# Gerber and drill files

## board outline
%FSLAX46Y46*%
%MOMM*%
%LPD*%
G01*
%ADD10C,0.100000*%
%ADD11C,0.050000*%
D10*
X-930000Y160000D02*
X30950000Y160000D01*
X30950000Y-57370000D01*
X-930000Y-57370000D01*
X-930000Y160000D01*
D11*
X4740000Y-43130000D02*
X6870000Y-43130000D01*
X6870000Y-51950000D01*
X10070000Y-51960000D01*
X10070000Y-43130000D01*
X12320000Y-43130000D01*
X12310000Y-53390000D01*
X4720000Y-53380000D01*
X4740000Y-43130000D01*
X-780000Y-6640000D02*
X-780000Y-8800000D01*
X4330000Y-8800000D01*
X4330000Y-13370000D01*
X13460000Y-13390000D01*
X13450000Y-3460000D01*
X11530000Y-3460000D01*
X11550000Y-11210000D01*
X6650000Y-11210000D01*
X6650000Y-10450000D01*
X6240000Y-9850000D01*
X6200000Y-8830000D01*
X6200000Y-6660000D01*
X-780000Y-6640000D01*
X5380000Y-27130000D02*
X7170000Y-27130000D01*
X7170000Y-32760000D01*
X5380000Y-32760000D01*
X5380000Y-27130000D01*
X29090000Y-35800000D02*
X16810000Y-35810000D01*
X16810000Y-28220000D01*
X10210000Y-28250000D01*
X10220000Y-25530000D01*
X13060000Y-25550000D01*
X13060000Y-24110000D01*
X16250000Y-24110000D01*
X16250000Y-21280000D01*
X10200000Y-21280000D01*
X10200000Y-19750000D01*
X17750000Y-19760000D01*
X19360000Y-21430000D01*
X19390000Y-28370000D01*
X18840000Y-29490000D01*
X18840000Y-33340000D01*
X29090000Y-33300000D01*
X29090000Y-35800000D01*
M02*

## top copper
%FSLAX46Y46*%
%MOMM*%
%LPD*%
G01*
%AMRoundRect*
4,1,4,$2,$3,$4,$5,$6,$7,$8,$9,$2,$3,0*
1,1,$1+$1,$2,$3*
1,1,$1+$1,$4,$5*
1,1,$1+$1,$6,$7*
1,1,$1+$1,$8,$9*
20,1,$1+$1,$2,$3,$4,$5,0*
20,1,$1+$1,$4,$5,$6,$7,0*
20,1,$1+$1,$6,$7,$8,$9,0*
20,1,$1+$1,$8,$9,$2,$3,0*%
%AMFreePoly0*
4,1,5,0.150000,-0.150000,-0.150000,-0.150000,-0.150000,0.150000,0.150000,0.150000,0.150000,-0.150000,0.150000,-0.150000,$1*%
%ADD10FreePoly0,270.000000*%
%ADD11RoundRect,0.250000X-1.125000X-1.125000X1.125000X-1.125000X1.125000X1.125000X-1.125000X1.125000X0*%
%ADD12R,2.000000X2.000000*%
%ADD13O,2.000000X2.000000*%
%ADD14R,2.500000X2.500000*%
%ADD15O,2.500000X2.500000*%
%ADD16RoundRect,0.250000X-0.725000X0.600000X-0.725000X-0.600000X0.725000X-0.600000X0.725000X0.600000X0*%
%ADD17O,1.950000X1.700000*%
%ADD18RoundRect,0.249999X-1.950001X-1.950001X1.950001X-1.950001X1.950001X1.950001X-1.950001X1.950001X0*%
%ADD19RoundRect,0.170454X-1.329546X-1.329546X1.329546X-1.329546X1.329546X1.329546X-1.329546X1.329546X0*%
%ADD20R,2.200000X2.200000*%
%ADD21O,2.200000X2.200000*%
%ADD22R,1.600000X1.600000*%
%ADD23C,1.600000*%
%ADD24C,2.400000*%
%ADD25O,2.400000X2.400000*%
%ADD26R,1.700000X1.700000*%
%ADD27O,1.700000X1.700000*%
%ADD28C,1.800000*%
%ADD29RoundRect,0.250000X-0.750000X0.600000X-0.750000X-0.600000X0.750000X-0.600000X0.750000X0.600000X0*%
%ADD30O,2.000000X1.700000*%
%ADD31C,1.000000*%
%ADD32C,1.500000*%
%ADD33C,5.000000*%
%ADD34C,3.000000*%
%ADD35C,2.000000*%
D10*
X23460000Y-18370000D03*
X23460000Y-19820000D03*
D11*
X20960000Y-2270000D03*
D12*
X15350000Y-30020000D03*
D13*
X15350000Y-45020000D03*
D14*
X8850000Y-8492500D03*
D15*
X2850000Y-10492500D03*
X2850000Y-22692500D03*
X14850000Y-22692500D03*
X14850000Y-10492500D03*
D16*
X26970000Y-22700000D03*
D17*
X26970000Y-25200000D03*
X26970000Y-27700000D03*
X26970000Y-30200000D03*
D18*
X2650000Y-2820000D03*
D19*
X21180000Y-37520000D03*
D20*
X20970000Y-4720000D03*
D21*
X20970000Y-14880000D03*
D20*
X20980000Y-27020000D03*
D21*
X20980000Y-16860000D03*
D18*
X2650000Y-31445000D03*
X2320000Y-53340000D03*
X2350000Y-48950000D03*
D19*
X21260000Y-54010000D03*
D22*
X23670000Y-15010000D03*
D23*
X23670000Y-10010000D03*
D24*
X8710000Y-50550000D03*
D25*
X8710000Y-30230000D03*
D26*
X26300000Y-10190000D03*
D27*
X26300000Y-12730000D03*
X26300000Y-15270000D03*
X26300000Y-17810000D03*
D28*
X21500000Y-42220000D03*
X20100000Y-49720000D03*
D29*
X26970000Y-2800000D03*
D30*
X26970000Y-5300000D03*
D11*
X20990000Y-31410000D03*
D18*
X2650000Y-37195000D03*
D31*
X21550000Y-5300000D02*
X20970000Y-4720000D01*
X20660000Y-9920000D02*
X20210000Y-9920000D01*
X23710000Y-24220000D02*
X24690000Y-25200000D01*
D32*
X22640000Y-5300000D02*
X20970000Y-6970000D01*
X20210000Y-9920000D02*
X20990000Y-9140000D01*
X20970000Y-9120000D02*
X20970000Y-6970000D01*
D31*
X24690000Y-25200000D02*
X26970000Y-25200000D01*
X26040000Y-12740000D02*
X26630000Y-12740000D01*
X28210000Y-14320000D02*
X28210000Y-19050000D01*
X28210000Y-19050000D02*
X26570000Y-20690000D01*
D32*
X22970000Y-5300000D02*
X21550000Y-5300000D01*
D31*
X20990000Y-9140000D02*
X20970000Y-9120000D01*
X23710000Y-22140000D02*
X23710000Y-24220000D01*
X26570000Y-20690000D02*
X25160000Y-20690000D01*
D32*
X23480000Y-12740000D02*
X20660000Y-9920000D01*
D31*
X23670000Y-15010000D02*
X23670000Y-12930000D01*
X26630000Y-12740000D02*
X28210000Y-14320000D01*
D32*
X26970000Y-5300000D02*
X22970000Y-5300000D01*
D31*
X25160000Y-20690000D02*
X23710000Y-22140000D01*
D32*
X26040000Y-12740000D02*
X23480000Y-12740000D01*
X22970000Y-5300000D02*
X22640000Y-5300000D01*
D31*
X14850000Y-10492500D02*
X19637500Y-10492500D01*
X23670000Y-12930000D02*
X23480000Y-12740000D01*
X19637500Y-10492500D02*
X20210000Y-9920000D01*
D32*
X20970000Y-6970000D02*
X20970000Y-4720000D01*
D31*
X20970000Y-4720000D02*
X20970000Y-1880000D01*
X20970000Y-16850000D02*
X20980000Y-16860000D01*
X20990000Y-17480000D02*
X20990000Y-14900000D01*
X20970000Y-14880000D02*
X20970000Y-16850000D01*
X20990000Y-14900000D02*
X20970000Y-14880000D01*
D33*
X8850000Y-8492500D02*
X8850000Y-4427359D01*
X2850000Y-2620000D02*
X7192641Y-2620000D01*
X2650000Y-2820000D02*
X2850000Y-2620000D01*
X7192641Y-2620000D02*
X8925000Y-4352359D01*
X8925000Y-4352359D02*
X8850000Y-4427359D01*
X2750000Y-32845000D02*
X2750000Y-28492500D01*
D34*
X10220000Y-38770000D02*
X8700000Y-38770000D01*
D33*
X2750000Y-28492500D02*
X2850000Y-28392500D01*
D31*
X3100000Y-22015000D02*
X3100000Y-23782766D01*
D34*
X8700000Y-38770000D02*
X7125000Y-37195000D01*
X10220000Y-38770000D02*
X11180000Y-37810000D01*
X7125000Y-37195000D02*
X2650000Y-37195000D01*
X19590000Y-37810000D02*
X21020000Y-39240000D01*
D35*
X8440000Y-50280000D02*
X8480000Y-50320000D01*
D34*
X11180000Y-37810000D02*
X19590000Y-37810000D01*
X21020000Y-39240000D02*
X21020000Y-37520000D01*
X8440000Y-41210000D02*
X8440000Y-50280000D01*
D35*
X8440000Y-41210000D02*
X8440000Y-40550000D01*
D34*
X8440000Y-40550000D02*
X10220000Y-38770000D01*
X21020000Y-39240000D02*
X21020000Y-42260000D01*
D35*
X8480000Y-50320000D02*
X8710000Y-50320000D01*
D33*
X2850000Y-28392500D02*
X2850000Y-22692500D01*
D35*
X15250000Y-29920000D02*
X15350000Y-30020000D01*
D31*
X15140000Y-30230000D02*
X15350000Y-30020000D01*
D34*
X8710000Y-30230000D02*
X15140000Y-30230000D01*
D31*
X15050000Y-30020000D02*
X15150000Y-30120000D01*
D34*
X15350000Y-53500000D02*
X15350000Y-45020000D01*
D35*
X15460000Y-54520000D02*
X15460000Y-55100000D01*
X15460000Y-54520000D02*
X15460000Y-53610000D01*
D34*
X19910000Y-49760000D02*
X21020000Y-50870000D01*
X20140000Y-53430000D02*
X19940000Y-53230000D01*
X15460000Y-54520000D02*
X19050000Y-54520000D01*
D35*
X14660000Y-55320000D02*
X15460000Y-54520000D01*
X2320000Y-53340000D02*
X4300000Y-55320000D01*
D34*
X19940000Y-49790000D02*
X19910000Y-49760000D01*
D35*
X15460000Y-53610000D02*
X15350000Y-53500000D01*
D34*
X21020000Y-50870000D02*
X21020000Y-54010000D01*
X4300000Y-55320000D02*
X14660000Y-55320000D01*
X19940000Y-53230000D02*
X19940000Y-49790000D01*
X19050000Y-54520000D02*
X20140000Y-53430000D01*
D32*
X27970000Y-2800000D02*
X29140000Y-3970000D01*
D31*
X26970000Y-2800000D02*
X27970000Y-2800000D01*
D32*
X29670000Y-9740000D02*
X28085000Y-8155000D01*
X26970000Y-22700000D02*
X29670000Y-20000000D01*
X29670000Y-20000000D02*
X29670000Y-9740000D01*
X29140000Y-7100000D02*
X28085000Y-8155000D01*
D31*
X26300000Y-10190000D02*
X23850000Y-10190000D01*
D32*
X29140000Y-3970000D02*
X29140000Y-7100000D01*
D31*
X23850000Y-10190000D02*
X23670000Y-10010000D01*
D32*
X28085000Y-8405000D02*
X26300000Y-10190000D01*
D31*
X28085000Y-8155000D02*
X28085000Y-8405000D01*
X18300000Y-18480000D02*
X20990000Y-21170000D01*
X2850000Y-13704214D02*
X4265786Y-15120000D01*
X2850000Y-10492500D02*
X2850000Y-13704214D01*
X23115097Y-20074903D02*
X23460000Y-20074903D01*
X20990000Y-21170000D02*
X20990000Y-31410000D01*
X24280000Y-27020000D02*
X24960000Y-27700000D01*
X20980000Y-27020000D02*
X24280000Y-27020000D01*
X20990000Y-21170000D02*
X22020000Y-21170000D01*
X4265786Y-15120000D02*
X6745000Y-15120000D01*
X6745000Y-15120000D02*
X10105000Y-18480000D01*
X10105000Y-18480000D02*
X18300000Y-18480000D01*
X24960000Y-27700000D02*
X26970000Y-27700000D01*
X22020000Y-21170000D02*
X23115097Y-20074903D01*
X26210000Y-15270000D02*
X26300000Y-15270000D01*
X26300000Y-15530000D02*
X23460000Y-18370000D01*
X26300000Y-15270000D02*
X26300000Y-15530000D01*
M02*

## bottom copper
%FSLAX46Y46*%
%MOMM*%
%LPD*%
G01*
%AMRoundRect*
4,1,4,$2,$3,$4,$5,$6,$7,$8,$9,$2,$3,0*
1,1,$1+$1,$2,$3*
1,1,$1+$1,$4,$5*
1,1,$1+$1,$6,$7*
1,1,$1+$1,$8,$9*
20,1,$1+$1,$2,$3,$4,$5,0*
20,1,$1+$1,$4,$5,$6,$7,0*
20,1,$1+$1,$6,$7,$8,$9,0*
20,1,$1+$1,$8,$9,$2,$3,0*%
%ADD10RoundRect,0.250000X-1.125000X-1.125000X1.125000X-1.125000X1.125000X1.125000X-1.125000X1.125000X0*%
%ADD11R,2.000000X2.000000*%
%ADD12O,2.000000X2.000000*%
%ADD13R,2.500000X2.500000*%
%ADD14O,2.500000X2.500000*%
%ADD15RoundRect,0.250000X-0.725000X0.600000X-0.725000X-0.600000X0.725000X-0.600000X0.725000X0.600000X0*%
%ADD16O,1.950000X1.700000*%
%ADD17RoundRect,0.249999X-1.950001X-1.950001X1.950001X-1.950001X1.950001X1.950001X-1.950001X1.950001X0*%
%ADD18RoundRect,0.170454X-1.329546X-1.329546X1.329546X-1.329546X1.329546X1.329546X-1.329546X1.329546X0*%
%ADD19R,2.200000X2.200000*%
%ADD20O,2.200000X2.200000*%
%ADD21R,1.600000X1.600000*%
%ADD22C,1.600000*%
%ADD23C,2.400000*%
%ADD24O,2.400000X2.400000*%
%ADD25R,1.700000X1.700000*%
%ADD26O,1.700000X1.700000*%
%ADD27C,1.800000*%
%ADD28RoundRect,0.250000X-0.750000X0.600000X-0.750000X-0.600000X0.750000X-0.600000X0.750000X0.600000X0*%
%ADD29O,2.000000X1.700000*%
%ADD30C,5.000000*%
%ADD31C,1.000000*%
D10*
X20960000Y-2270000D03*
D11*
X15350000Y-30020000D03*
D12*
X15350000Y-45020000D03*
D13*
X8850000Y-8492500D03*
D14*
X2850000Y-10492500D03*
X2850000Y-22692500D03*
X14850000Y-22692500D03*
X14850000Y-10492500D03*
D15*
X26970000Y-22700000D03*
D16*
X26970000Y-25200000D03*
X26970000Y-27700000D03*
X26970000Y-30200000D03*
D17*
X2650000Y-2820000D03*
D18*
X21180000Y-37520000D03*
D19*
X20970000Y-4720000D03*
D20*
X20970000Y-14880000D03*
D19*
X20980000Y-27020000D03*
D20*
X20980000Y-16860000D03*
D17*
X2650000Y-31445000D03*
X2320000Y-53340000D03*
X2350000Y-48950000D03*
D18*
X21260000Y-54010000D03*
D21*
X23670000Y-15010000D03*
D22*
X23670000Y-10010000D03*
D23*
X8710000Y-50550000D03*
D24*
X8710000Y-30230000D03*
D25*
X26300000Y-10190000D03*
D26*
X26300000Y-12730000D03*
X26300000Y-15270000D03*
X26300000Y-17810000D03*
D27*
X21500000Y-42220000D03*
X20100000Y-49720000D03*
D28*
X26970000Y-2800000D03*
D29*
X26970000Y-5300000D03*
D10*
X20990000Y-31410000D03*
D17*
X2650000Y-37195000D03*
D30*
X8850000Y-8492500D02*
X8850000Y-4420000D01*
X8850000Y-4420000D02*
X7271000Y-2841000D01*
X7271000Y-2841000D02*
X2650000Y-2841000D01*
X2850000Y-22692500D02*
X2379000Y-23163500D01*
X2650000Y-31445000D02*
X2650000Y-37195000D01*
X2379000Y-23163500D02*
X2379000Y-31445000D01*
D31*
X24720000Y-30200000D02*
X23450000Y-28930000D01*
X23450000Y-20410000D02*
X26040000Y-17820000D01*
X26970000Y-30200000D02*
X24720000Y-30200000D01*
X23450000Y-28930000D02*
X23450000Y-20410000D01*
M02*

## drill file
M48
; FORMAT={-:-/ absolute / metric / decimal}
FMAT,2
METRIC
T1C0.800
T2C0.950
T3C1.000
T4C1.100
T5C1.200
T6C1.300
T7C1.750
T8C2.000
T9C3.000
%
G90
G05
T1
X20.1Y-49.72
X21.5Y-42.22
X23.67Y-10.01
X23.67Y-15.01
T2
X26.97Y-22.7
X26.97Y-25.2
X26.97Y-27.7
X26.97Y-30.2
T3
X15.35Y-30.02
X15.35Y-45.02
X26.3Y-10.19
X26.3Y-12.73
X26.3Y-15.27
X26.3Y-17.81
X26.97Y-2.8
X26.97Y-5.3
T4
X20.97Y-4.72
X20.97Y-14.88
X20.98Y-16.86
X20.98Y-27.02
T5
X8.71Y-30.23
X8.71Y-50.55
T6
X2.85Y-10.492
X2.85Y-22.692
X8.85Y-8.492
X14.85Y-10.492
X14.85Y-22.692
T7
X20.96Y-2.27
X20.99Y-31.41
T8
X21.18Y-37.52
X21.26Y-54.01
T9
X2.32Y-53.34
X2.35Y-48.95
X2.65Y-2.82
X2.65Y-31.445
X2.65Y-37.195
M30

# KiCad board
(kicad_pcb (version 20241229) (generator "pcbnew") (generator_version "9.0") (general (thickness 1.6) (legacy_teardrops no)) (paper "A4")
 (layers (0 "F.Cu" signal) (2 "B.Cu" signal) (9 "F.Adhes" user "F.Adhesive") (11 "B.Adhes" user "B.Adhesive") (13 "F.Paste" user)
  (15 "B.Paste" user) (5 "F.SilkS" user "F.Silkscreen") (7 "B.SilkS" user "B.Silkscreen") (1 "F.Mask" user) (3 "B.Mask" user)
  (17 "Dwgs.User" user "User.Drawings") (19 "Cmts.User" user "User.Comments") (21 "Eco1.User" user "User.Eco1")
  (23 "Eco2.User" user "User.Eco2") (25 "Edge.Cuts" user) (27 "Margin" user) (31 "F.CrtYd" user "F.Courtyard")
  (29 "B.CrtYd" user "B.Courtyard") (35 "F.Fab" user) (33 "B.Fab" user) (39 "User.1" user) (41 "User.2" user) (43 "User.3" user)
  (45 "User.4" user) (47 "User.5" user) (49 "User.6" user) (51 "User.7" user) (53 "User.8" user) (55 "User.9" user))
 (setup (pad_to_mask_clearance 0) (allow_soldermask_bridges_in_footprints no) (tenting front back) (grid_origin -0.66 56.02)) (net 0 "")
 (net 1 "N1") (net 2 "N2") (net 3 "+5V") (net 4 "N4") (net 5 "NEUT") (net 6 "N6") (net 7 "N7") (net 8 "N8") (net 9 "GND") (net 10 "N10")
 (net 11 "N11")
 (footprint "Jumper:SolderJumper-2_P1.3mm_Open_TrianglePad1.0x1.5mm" (layer "F.Cu") (at 23.46 19.095 -90)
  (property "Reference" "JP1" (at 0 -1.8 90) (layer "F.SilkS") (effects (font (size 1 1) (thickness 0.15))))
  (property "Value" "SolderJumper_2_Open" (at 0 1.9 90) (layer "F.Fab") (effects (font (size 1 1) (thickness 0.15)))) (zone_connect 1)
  (pad "1" smd custom (at -0.725 0 270) (size 0.3 0.3) (layers "F.Cu" "F.Mask") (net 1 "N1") (zone_connect 2) (thermal_bridge_angle 45)
   (options (clearance outline) (anchor rect)) (primitives))
  (pad "2" smd custom (at 0.725 0 270) (size 0.3 0.3) (layers "F.Cu" "F.Mask") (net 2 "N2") (zone_connect 2) (thermal_bridge_angle 45)
   (options (clearance outline) (anchor rect)) (primitives)))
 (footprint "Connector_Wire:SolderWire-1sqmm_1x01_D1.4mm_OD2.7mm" (layer "F.Cu") (at 20.96 2.27)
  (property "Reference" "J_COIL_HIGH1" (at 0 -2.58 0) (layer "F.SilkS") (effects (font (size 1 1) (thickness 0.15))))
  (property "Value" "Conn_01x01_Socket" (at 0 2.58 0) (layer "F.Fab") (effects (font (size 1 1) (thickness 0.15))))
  (pad "1" thru_hole roundrect (at 0 0) (size 2.75 2.75) (drill 1.75) (layers "*.Cu" "*.Mask") (remove_unused_layers no)
   (roundrect_rratio 0.090909) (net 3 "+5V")))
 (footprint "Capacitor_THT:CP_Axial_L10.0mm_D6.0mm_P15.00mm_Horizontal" (layer "F.Cu") (at 15.35 30.02 -90)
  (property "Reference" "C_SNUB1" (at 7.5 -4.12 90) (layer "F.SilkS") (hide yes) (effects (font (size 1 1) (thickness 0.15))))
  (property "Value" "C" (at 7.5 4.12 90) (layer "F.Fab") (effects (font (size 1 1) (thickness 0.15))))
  (pad "1" thru_hole rect (at 0 0 270) (size 2 2) (drill 1) (layers "*.Cu" "*.Mask") (remove_unused_layers no) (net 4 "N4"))
  (pad "2" thru_hole oval (at 15 0 270) (size 2 2) (drill 1) (layers "*.Cu" "*.Mask") (remove_unused_layers no) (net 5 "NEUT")))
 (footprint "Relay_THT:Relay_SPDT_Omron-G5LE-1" (layer "F.Cu") (at 8.85 8.4925)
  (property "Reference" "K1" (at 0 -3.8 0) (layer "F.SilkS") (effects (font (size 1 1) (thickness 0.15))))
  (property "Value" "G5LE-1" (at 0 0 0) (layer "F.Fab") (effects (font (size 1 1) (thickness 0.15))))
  (pad "1" thru_hole rect (at 0 0) (size 2.5 2.5) (drill 1.3) (layers "*.Cu" "*.Mask") (remove_unused_layers no) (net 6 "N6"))
  (pad "2" thru_hole oval (at -6 2) (size 2.5 2.5) (drill 1.3) (layers "*.Cu" "*.Mask") (remove_unused_layers no) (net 2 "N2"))
  (pad "3" thru_hole oval (at -6 14.2) (size 2.5 2.5) (drill 1.3) (layers "*.Cu" "*.Mask") (remove_unused_layers no) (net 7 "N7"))
  (pad "4" thru_hole oval (at 6 14.2) (size 2.5 2.5) (drill 1.3) (layers "*.Cu" "*.Mask") (remove_unused_layers no) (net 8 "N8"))
  (pad "5" thru_hole oval (at 6 2) (size 2.5 2.5) (drill 1.3) (layers "*.Cu" "*.Mask") (remove_unused_layers no) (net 3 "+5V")))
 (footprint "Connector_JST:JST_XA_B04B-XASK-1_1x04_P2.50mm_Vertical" (layer "F.Cu") (at 26.97 22.7 -90)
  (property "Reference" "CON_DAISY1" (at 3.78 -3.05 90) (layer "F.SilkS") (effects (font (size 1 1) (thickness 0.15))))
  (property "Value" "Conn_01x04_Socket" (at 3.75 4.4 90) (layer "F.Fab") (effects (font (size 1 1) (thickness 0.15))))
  (pad "1" thru_hole roundrect (at 0 0 270) (size 1.7 1.95) (drill 0.95) (layers "*.Cu" "*.Mask") (remove_unused_layers no)
   (roundrect_rratio 0.147059) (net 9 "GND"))
  (pad "2" thru_hole oval (at 2.5 0 270) (size 1.7 1.95) (drill 0.95) (layers "*.Cu" "*.Mask") (remove_unused_layers no) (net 3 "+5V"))
  (pad "3" thru_hole oval (at 5 0 270) (size 1.7 1.95) (drill 0.95) (layers "*.Cu" "*.Mask") (remove_unused_layers no) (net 2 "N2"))
  (pad "4" thru_hole oval (at 7.5 0 270) (size 1.7 1.95) (drill 0.95) (layers "*.Cu" "*.Mask") (remove_unused_layers no) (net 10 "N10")))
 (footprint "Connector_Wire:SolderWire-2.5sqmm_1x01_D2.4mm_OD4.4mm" (layer "F.Cu") (at 2.65 2.82)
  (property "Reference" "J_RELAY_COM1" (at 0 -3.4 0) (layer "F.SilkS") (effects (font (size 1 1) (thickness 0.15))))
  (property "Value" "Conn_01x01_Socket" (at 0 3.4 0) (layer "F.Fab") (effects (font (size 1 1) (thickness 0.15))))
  (pad "1" thru_hole roundrect (at 0 0) (size 4.4 4.4) (drill 3) (layers "*.Cu" "*.Mask") (remove_unused_layers no)
   (roundrect_rratio 0.056818) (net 6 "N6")))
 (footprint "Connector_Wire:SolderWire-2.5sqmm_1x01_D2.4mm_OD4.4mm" (layer "F.Cu") (at 21.18 37.52)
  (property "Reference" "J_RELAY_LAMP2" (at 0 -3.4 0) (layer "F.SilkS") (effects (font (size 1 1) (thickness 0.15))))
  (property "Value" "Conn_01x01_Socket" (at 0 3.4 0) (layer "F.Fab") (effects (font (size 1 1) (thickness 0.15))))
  (pad "1" thru_hole roundrect (at 0 0) (size 3 3) (drill 2) (layers "*.Cu" "*.Mask") (remove_unused_layers no) (roundrect_rratio 0.056818)
   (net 7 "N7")))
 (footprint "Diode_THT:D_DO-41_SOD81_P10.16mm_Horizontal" (layer "F.Cu") (at 20.97 4.72 -90)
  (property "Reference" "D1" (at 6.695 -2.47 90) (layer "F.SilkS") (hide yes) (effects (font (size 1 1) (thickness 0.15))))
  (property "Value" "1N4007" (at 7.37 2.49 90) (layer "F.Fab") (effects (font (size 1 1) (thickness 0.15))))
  (pad "1" thru_hole rect (at 0 0 270) (size 2.2 2.2) (drill 1.1) (layers "*.Cu" "*.Mask") (remove_unused_layers no) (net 3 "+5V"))
  (pad "2" thru_hole oval (at 10.16 0 270) (size 2.2 2.2) (drill 1.1) (layers "*.Cu" "*.Mask") (remove_unused_layers no) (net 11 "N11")))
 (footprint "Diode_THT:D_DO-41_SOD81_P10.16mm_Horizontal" (layer "F.Cu") (at 20.98 27.02 90)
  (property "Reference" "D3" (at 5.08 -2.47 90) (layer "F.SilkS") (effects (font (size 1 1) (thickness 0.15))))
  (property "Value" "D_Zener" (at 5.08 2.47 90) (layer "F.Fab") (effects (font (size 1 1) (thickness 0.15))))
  (pad "1" thru_hole rect (at 0 0 90) (size 2.2 2.2) (drill 1.1) (layers "*.Cu" "*.Mask") (remove_unused_layers no) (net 2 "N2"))
  (pad "2" thru_hole oval (at 10.16 0 90) (size 2.2 2.2) (drill 1.1) (layers "*.Cu" "*.Mask") (remove_unused_layers no) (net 11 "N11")))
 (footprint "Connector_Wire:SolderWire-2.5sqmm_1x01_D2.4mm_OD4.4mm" (layer "F.Cu") (at 2.65 31.445)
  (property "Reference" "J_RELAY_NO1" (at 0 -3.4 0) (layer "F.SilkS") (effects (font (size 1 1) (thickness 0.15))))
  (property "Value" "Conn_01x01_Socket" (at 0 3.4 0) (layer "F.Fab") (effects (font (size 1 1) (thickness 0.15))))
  (pad "1" thru_hole roundrect (at 0 0) (size 4.4 4.4) (drill 3) (layers "*.Cu" "*.Mask") (remove_unused_layers no)
   (roundrect_rratio 0.056818) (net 7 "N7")))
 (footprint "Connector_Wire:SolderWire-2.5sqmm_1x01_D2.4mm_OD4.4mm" (layer "F.Cu") (at 2.32 53.34)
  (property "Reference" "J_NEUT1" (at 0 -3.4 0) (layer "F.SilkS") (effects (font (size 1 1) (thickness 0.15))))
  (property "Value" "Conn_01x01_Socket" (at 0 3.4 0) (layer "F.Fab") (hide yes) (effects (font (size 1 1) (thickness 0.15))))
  (pad "1" thru_hole roundrect (at 0 0) (size 4.4 4.4) (drill 3) (layers "*.Cu" "*.Mask") (remove_unused_layers no)
   (roundrect_rratio 0.056818) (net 5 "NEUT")))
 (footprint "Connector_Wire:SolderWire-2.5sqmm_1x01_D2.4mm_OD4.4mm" (layer "F.Cu") (at 2.35 48.95)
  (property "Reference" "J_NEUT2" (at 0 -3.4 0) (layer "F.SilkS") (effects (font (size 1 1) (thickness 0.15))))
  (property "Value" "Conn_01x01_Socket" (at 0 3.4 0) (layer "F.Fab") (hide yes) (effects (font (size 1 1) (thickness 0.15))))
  (pad "1" thru_hole roundrect (at 0 0) (size 4.4 4.4) (drill 3) (layers "*.Cu" "*.Mask") (remove_unused_layers no)
   (roundrect_rratio 0.056818) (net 5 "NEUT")))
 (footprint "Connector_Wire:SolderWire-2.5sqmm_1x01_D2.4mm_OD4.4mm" (layer "F.Cu") (at 21.26 54.01)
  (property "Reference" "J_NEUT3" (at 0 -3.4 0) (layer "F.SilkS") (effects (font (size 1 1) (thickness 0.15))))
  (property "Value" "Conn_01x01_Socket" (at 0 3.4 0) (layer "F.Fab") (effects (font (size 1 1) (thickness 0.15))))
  (pad "1" thru_hole roundrect (at 0 0) (size 3 3) (drill 2) (layers "*.Cu" "*.Mask") (remove_unused_layers no) (roundrect_rratio 0.056818)
   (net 5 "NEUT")))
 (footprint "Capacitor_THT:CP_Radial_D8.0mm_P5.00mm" (layer "F.Cu") (at 23.67 15.01 90)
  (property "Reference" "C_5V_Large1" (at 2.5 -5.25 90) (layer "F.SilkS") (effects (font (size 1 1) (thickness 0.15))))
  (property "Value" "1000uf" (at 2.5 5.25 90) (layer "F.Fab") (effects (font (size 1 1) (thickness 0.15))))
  (pad "1" thru_hole rect (at 0 0 90) (size 1.6 1.6) (drill 0.8) (layers "*.Cu" "*.Mask") (remove_unused_layers no) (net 3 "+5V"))
  (pad "2" thru_hole circle (at 5 0 90) (size 1.6 1.6) (drill 0.8) (layers "*.Cu" "*.Mask") (remove_unused_layers no) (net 9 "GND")))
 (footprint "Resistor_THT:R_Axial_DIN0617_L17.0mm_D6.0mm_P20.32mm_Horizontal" (layer "F.Cu") (at 8.71 50.55 90)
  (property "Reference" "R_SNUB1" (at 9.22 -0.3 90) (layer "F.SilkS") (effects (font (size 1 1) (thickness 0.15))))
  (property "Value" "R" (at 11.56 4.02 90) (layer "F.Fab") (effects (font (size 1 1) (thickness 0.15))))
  (pad "1" thru_hole circle (at 0 0 90) (size 2.4 2.4) (drill 1.2) (layers "*.Cu" "*.Mask") (remove_unused_layers no) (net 7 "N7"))
  (pad "2" thru_hole oval (at 20.32 0 90) (size 2.4 2.4) (drill 1.2) (layers "*.Cu" "*.Mask") (remove_unused_layers no) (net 4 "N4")))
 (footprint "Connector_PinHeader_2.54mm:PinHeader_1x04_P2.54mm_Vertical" (layer "F.Cu") (at 26.3 10.19)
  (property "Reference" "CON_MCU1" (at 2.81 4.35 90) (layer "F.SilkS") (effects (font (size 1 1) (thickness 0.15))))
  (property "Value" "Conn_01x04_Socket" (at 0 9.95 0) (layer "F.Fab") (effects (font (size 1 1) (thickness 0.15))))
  (pad "1" thru_hole rect (at 0 0) (size 1.7 1.7) (drill 1) (layers "*.Cu" "*.Mask") (remove_unused_layers no) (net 9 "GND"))
  (pad "2" thru_hole oval (at 0 2.54) (size 1.7 1.7) (drill 1) (layers "*.Cu" "*.Mask") (remove_unused_layers no) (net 3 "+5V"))
  (pad "3" thru_hole oval (at 0 5.08) (size 1.7 1.7) (drill 1) (layers "*.Cu" "*.Mask") (remove_unused_layers no) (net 1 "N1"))
  (pad "4" thru_hole oval (at 0 7.62) (size 1.7 1.7) (drill 1) (layers "*.Cu" "*.Mask") (remove_unused_layers no) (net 10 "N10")))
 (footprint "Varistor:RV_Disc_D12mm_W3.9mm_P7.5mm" (layer "F.Cu") (at 21.5 42.22 -90)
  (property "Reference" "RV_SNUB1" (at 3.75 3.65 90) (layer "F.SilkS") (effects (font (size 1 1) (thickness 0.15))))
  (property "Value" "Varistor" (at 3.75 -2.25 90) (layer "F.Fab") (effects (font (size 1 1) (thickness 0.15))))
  (pad "1" thru_hole circle (at 0 0 270) (size 1.8 1.8) (drill 0.8) (layers "*.Cu" "*.Mask") (remove_unused_layers no) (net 7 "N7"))
  (pad "2" thru_hole circle (at 7.5 1.4 270) (size 1.8 1.8) (drill 0.8) (layers "*.Cu" "*.Mask") (remove_unused_layers no) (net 5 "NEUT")))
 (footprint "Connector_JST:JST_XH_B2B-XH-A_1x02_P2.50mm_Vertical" (layer "F.Cu") (at 26.97 2.8 -90)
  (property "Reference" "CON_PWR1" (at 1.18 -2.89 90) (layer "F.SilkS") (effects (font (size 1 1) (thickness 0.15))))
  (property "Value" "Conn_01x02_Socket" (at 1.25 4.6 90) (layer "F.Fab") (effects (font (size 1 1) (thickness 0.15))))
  (pad "1" thru_hole roundrect (at 0 0 270) (size 1.7 2) (drill 1) (layers "*.Cu" "*.Mask") (remove_unused_layers no)
   (roundrect_rratio 0.147059) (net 9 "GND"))
  (pad "2" thru_hole oval (at 2.5 0 270) (size 1.7 2) (drill 1) (layers "*.Cu" "*.Mask") (remove_unused_layers no) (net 3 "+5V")))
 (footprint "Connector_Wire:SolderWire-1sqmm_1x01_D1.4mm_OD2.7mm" (layer "F.Cu") (at 20.99 31.41)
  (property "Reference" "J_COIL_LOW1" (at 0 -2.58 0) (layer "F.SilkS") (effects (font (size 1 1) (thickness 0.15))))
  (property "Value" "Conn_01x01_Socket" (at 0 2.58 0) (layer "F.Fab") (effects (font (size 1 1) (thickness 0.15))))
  (pad "1" thru_hole roundrect (at 0 0) (size 2.75 2.75) (drill 1.75) (layers "*.Cu" "*.Mask") (remove_unused_layers no)
   (roundrect_rratio 0.090909) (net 2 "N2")))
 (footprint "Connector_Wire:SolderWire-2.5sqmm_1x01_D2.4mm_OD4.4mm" (layer "F.Cu") (at 2.65 37.195)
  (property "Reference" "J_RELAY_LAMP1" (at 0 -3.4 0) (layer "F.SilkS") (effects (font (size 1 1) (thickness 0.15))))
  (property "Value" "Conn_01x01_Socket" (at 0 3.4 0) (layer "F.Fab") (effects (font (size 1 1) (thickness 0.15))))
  (pad "1" thru_hole roundrect (at 0 0) (size 4.4 4.4) (drill 3) (layers "*.Cu" "*.Mask") (remove_unused_layers no)
   (roundrect_rratio 0.056818) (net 7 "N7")))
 (gr_rect (start -0.93 -0.16) (end 30.95 57.37) (stroke (width 0.1) (type default)) (fill no) (layer "Edge.Cuts"))
 (gr_poly
  (pts (xy 4.74 43.13) (xy 6.87 43.13) (xy 6.87 51.95) (xy 10.07 51.96) (xy 10.07 43.13) (xy 12.32 43.13) (xy 12.31 53.39) (xy 4.72 53.38))
  (stroke (width 0.05) (type solid)) (fill no) (layer "Edge.Cuts"))
 (gr_poly
  (pts (xy -0.78 6.64) (xy -0.78 8.8) (xy 4.33 8.8) (xy 4.33 13.37) (xy 13.46 13.39) (xy 13.45 3.46) (xy 11.53 3.46) (xy 11.55 11.21)
   (xy 6.65 11.21) (xy 6.65 10.45) (xy 6.24 9.85) (xy 6.2 8.83) (xy 6.2 6.66))
  (stroke (width 0.05) (type solid)) (fill no) (layer "Edge.Cuts"))
 (gr_rect (start 5.38 27.13) (end 7.17 32.76) (stroke (width 0.05) (type solid)) (fill no) (layer "Edge.Cuts"))
 (gr_poly
  (pts (xy 29.09 35.8) (xy 16.81 35.81) (xy 16.81 28.22) (xy 10.21 28.25) (xy 10.22 25.53) (xy 13.06 25.55) (xy 13.06 24.11)
   (xy 16.25 24.11) (xy 16.25 21.28) (xy 10.2 21.28) (xy 10.2 19.75) (xy 17.75 19.76) (xy 19.36 21.43) (xy 19.39 28.37) (xy 18.84 29.49)
   (xy 18.84 33.34) (xy 29.09 33.3))
  (stroke (width 0.05) (type solid)) (fill no) (layer "Edge.Cuts"))
 (segment (start 21.55 5.3) (end 20.97 4.72) (width 1) (layer "F.Cu") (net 3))
 (segment (start 20.66 9.92) (end 20.21 9.92) (width 1) (layer "F.Cu") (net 3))
 (segment (start 23.71 24.22) (end 24.69 25.2) (width 1) (layer "F.Cu") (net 3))
 (segment (start 22.64 5.3) (end 20.97 6.97) (width 1.5) (layer "F.Cu") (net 3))
 (segment (start 20.21 9.92) (end 20.99 9.14) (width 1.5) (layer "F.Cu") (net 3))
 (segment (start 20.97 9.12) (end 20.97 6.97) (width 1.5) (layer "F.Cu") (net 3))
 (segment (start 24.69 25.2) (end 26.97 25.2) (width 1) (layer "F.Cu") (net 3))
 (segment (start 26.04 12.74) (end 26.63 12.74) (width 1) (layer "F.Cu") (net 3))
 (segment (start 28.21 14.32) (end 28.21 19.05) (width 1) (layer "F.Cu") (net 3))
 (segment (start 28.21 19.05) (end 26.57 20.69) (width 1) (layer "F.Cu") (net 3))
 (segment (start 22.97 5.3) (end 21.55 5.3) (width 1.5) (layer "F.Cu") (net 3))
 (segment (start 20.99 9.14) (end 20.97 9.12) (width 1) (layer "F.Cu") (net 3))
 (segment (start 23.71 22.14) (end 23.71 24.22) (width 1) (layer "F.Cu") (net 3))
 (segment (start 26.57 20.69) (end 25.16 20.69) (width 1) (layer "F.Cu") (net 3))
 (segment (start 23.48 12.74) (end 20.66 9.92) (width 1.5) (layer "F.Cu") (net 3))
 (segment (start 23.67 15.01) (end 23.67 12.93) (width 1) (layer "F.Cu") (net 3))
 (segment (start 26.63 12.74) (end 28.21 14.32) (width 1) (layer "F.Cu") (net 3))
 (segment (start 26.97 5.3) (end 22.97 5.3) (width 1.5) (layer "F.Cu") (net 3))
 (segment (start 25.16 20.69) (end 23.71 22.14) (width 1) (layer "F.Cu") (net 3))
 (segment (start 26.04 12.74) (end 23.48 12.74) (width 1.5) (layer "F.Cu") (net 3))
 (segment (start 22.97 5.3) (end 22.64 5.3) (width 1.5) (layer "F.Cu") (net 3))
 (segment (start 14.85 10.4925) (end 19.6375 10.4925) (width 1) (layer "F.Cu") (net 3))
 (segment (start 23.67 12.93) (end 23.48 12.74) (width 1) (layer "F.Cu") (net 3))
 (segment (start 19.6375 10.4925) (end 20.21 9.92) (width 1) (layer "F.Cu") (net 3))
 (segment (start 20.97 6.97) (end 20.97 4.72) (width 1.5) (layer "F.Cu") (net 3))
 (segment (start 20.97 4.72) (end 20.97 1.88) (width 1) (layer "F.Cu") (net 3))
 (segment (start 20.97 16.85) (end 20.98 16.86) (width 1) (layer "F.Cu") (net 11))
 (segment (start 20.99 17.48) (end 20.99 14.9) (width 1) (layer "F.Cu") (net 11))
 (segment (start 20.97 14.88) (end 20.97 16.85) (width 1) (layer "F.Cu") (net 11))
 (segment (start 20.99 14.9) (end 20.97 14.88) (width 1) (layer "F.Cu") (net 11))
 (segment (start 8.85 8.4925) (end 8.85 4.427359) (width 5) (layer "F.Cu") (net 6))
 (segment (start 2.85 2.62) (end 7.192641 2.62) (width 5) (layer "F.Cu") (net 6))
 (segment (start 2.65 2.82) (end 2.85 2.62) (width 5) (layer "F.Cu") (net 6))
 (segment (start 7.192641 2.62) (end 8.925 4.352359) (width 5) (layer "F.Cu") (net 6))
 (segment (start 8.925 4.352359) (end 8.85 4.427359) (width 5) (layer "F.Cu") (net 6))
 (segment (start 8.85 8.4925) (end 8.85 4.42) (width 5) (layer "B.Cu") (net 6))
 (segment (start 8.85 4.42) (end 7.271 2.841) (width 5) (layer "B.Cu") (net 6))
 (segment (start 7.271 2.841) (end 2.65 2.841) (width 5) (layer "B.Cu") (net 6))
 (segment (start 2.75 32.845) (end 2.75 28.4925) (width 5) (layer "F.Cu") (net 7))
 (segment (start 10.22 38.77) (end 8.7 38.77) (width 3) (layer "F.Cu") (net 7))
 (segment (start 2.75 28.4925) (end 2.85 28.3925) (width 5) (layer "F.Cu") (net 7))
 (segment (start 3.1 22.015) (end 3.1 23.782766) (width 1) (layer "F.Cu") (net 7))
 (segment (start 8.7 38.77) (end 7.125 37.195) (width 3) (layer "F.Cu") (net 7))
 (segment (start 10.22 38.77) (end 11.18 37.81) (width 3) (layer "F.Cu") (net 7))
 (segment (start 7.125 37.195) (end 2.65 37.195) (width 3) (layer "F.Cu") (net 7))
 (segment (start 19.59 37.81) (end 21.02 39.24) (width 3) (layer "F.Cu") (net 7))
 (segment (start 8.44 50.28) (end 8.48 50.32) (width 2) (layer "F.Cu") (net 7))
 (segment (start 11.18 37.81) (end 19.59 37.81) (width 3) (layer "F.Cu") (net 7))
 (segment (start 21.02 39.24) (end 21.02 37.52) (width 3) (layer "F.Cu") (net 7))
 (segment (start 8.44 41.21) (end 8.44 50.28) (width 3) (layer "F.Cu") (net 7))
 (segment (start 8.44 41.21) (end 8.44 40.55) (width 2) (layer "F.Cu") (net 7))
 (segment (start 8.44 40.55) (end 10.22 38.77) (width 3) (layer "F.Cu") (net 7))
 (segment (start 21.02 39.24) (end 21.02 42.26) (width 3) (layer "F.Cu") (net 7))
 (segment (start 8.48 50.32) (end 8.71 50.32) (width 2) (layer "F.Cu") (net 7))
 (segment (start 2.85 28.3925) (end 2.85 22.6925) (width 5) (layer "F.Cu") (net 7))
 (segment (start 2.85 22.6925) (end 2.379 23.1635) (width 5) (layer "B.Cu") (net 7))
 (segment (start 2.65 31.445) (end 2.65 37.195) (width 5) (layer "B.Cu") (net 7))
 (segment (start 2.379 23.1635) (end 2.379 31.445) (width 5) (layer "B.Cu") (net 7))
 (segment (start 15.25 29.92) (end 15.35 30.02) (width 2) (layer "F.Cu") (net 4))
 (segment (start 15.14 30.23) (end 15.35 30.02) (width 1) (layer "F.Cu") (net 4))
 (segment (start 8.71 30.23) (end 15.14 30.23) (width 3) (layer "F.Cu") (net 4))
 (segment (start 15.05 30.02) (end 15.15 30.12) (width 1) (layer "F.Cu") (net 4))
 (segment (start 15.35 53.5) (end 15.35 45.02) (width 3) (layer "F.Cu") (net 5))
 (segment (start 15.46 54.52) (end 15.46 55.1) (width 2) (layer "F.Cu") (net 5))
 (segment (start 15.46 54.52) (end 15.46 53.61) (width 2) (layer "F.Cu") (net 5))
 (segment (start 19.91 49.76) (end 21.02 50.87) (width 3) (layer "F.Cu") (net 5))
 (segment (start 20.14 53.43) (end 19.94 53.23) (width 3) (layer "F.Cu") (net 5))
 (segment (start 15.46 54.52) (end 19.05 54.52) (width 3) (layer "F.Cu") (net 5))
 (segment (start 14.66 55.32) (end 15.46 54.52) (width 2) (layer "F.Cu") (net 5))
 (segment (start 2.32 53.34) (end 4.3 55.32) (width 2) (layer "F.Cu") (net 5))
 (segment (start 19.94 49.79) (end 19.91 49.76) (width 3) (layer "F.Cu") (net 5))
 (segment (start 15.46 53.61) (end 15.35 53.5) (width 2) (layer "F.Cu") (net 5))
 (segment (start 21.02 50.87) (end 21.02 54.01) (width 3) (layer "F.Cu") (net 5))
 (segment (start 4.3 55.32) (end 14.66 55.32) (width 3) (layer "F.Cu") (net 5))
 (segment (start 19.94 53.23) (end 19.94 49.79) (width 3) (layer "F.Cu") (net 5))
 (segment (start 19.05 54.52) (end 20.14 53.43) (width 3) (layer "F.Cu") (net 5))
 (segment (start 27.97 2.8) (end 29.14 3.97) (width 1.5) (layer "F.Cu") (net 9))
 (segment (start 26.97 2.8) (end 27.97 2.8) (width 1) (layer "F.Cu") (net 9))
 (segment (start 29.67 9.74) (end 28.085 8.155) (width 1.5) (layer "F.Cu") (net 9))
 (segment (start 26.97 22.7) (end 29.67 20) (width 1.5) (layer "F.Cu") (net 9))
 (segment (start 29.67 20) (end 29.67 9.74) (width 1.5) (layer "F.Cu") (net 9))
 (segment (start 29.14 7.1) (end 28.085 8.155) (width 1.5) (layer "F.Cu") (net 9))
 (segment (start 26.3 10.19) (end 23.85 10.19) (width 1) (layer "F.Cu") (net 9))
 (segment (start 29.14 3.97) (end 29.14 7.1) (width 1.5) (layer "F.Cu") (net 9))
 (segment (start 23.85 10.19) (end 23.67 10.01) (width 1) (layer "F.Cu") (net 9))
 (segment (start 28.085 8.405) (end 26.3 10.19) (width 1.5) (layer "F.Cu") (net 9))
 (segment (start 28.085 8.155) (end 28.085 8.405) (width 1) (layer "F.Cu") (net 9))
 (segment (start 24.72 30.2) (end 23.45 28.93) (width 1) (layer "B.Cu") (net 10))
 (segment (start 23.45 20.41) (end 26.04 17.82) (width 1) (layer "B.Cu") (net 10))
 (segment (start 26.97 30.2) (end 24.72 30.2) (width 1) (layer "B.Cu") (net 10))
 (segment (start 23.45 28.93) (end 23.45 20.41) (width 1) (layer "B.Cu") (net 10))
 (segment (start 18.3 18.48) (end 20.99 21.17) (width 1) (layer "F.Cu") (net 2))
 (segment (start 2.85 13.704214) (end 4.265786 15.12) (width 1) (layer "F.Cu") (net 2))
 (segment (start 2.85 10.4925) (end 2.85 13.704214) (width 1) (layer "F.Cu") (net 2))
 (segment (start 23.115097 20.074903) (end 23.46 20.074903) (width 1) (layer "F.Cu") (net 2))
 (segment (start 20.99 21.17) (end 20.99 31.41) (width 1) (layer "F.Cu") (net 2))
 (segment (start 24.28 27.02) (end 24.96 27.7) (width 1) (layer "F.Cu") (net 2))
 (segment (start 20.98 27.02) (end 24.28 27.02) (width 1) (layer "F.Cu") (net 2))
 (segment (start 20.99 21.17) (end 22.02 21.17) (width 1) (layer "F.Cu") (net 2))
 (segment (start 4.265786 15.12) (end 6.745 15.12) (width 1) (layer "F.Cu") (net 2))
 (segment (start 6.745 15.12) (end 10.105 18.48) (width 1) (layer "F.Cu") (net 2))
 (segment (start 10.105 18.48) (end 18.3 18.48) (width 1) (layer "F.Cu") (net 2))
 (segment (start 24.96 27.7) (end 26.97 27.7) (width 1) (layer "F.Cu") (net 2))
 (segment (start 22.02 21.17) (end 23.115097 20.074903) (width 1) (layer "F.Cu") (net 2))
 (segment (start 26.21 15.27) (end 26.3 15.27) (width 1) (layer "F.Cu") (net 1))
 (segment (start 26.3 15.53) (end 23.46 18.37) (width 1) (layer "F.Cu") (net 1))
 (segment (start 26.3 15.27) (end 26.3 15.53) (width 1) (layer "F.Cu") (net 1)))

